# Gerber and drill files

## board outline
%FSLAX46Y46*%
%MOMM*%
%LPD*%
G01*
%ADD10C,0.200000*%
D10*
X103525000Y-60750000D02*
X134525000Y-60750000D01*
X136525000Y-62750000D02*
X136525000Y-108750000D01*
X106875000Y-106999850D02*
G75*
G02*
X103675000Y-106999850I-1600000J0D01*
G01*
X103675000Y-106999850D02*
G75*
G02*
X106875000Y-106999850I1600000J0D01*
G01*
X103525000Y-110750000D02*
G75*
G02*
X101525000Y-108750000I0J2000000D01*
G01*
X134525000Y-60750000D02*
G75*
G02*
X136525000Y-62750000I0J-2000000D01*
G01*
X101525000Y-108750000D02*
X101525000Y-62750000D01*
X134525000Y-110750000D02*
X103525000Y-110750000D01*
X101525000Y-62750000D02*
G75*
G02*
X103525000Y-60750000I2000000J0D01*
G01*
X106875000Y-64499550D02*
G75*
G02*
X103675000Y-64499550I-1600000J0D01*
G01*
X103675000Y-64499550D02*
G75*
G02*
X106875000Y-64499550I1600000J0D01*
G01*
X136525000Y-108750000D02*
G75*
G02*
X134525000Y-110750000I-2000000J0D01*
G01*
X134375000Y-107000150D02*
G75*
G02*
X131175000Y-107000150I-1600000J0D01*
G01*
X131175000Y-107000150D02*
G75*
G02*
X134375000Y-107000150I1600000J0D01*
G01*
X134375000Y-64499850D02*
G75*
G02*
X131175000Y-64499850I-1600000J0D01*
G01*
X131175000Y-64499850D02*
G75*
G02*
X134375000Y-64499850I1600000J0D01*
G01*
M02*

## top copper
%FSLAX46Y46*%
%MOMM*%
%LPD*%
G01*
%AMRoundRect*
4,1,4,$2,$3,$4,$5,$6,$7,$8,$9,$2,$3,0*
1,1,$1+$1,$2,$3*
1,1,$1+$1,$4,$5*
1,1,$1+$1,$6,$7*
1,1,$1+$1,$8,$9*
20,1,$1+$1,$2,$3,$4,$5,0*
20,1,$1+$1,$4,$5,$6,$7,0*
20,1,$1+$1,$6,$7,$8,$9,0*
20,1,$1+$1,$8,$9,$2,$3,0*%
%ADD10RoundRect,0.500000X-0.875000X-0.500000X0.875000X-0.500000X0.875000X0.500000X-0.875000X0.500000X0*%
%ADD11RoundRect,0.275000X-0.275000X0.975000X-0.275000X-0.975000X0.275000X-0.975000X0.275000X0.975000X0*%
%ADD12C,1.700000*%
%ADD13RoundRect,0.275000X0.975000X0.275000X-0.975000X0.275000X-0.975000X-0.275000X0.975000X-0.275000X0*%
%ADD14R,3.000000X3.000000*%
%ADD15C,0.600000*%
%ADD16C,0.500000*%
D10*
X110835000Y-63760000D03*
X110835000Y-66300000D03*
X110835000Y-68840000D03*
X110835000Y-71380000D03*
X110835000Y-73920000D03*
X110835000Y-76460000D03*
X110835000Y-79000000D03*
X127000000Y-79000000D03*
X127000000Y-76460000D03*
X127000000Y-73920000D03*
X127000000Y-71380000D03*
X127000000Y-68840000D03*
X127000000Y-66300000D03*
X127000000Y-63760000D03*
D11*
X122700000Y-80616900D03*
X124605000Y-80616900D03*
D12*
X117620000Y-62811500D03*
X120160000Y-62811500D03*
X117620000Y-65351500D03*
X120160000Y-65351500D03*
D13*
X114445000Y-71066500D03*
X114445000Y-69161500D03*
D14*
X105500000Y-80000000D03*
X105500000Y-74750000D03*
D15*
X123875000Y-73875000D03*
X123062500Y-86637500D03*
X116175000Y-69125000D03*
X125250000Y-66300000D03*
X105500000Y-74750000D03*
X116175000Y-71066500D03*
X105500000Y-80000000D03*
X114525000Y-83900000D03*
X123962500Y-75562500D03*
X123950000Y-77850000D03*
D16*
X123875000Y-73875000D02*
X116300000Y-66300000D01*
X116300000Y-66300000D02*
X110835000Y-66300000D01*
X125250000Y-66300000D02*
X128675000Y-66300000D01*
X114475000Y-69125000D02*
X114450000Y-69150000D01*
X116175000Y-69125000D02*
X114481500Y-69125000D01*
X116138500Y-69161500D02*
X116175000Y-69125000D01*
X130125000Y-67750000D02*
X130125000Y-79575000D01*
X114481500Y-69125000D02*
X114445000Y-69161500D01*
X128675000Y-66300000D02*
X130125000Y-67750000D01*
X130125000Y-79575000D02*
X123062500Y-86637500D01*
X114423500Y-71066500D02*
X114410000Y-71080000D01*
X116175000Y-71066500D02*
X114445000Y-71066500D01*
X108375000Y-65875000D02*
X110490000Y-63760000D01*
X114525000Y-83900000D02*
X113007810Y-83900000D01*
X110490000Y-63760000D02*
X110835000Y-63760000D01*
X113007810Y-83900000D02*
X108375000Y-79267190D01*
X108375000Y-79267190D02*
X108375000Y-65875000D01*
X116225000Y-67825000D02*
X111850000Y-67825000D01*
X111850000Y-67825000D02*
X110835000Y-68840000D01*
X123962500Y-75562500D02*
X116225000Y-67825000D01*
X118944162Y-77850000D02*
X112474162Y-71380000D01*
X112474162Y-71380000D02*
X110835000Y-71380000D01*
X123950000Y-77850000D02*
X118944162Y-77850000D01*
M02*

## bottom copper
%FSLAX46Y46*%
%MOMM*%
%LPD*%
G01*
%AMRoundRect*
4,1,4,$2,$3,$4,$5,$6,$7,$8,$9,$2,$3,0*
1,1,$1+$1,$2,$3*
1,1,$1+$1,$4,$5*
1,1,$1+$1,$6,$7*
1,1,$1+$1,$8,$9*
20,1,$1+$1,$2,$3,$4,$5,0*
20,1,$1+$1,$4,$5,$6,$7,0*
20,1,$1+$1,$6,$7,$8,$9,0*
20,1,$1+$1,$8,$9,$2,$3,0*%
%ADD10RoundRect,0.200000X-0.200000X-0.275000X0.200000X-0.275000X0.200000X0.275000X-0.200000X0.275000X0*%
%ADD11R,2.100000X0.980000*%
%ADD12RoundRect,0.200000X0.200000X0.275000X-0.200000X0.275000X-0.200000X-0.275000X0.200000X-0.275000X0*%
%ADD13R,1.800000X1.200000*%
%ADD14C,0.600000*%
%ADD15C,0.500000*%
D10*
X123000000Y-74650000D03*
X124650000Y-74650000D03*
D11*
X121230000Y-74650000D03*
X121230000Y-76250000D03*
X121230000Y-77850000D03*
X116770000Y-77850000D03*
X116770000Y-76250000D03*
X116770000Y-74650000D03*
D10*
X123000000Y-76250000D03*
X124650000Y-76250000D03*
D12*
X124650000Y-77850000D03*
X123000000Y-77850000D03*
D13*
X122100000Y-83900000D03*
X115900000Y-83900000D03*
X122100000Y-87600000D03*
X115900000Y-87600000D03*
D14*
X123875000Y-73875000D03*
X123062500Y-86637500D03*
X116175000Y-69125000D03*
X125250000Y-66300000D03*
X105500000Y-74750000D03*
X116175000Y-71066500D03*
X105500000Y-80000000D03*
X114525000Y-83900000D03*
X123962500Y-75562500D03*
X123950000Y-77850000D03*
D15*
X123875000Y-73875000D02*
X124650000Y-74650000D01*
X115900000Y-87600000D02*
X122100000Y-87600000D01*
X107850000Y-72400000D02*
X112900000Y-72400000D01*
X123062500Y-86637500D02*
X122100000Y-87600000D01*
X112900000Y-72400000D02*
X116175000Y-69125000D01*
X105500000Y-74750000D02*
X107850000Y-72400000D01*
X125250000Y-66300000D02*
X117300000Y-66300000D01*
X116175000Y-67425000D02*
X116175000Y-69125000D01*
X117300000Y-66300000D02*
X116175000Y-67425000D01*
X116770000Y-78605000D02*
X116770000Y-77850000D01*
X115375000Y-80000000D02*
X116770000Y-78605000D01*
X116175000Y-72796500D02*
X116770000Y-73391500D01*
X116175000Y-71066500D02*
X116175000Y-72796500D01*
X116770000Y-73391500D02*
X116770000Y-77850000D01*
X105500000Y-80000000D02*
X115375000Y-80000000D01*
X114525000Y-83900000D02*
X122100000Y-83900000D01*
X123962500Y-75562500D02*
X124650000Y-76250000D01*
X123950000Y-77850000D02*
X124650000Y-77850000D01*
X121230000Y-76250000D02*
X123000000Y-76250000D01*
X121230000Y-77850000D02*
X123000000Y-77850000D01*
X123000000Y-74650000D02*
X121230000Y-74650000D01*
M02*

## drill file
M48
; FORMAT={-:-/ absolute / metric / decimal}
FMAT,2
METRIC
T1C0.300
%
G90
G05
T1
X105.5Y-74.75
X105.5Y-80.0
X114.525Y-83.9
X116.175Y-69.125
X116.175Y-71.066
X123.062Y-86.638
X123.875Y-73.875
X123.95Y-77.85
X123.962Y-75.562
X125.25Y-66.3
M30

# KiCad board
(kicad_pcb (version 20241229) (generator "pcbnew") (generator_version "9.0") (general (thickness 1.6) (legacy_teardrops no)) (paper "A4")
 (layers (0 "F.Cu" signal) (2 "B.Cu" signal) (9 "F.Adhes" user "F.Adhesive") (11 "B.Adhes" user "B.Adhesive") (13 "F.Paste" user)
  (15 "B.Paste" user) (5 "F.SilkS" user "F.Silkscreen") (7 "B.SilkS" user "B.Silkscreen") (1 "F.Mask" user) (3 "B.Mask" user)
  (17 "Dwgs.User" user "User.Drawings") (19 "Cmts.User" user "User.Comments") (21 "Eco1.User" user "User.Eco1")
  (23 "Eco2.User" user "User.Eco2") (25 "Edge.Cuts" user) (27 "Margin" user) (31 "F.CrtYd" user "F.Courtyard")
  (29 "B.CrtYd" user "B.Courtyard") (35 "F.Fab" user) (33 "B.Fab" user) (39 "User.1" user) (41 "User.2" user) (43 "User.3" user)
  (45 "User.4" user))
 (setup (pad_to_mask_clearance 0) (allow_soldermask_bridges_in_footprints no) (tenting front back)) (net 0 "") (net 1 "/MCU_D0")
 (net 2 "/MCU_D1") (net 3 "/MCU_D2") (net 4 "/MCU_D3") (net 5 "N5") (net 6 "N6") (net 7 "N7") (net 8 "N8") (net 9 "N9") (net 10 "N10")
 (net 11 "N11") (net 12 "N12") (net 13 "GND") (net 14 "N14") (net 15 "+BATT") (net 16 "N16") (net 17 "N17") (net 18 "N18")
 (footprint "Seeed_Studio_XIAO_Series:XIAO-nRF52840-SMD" (layer "F.Cu") (at 110 81.88)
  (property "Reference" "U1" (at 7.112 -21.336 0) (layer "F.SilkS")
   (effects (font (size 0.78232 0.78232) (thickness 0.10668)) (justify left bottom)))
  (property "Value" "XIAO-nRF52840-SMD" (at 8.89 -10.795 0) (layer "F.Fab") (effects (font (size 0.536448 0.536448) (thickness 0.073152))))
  (pad "1" smd roundrect (at 0.835 -18.12) (size 2.75 2) (layers "F.Cu" "F.Mask" "F.Paste") (roundrect_rratio 0.25) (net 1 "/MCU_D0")
   (solder_mask_margin 0.0508) (thermal_bridge_angle 45))
  (pad "2" smd roundrect (at 0.835 -15.58) (size 2.75 2) (layers "F.Cu" "F.Mask" "F.Paste") (roundrect_rratio 0.25) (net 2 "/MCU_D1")
   (solder_mask_margin 0.0508) (thermal_bridge_angle 45))
  (pad "3" smd roundrect (at 0.835 -13.04) (size 2.75 2) (layers "F.Cu" "F.Mask" "F.Paste") (roundrect_rratio 0.25) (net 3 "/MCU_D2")
   (solder_mask_margin 0.0508) (thermal_bridge_angle 45))
  (pad "4" smd roundrect (at 0.835 -10.5) (size 2.75 2) (layers "F.Cu" "F.Mask" "F.Paste") (roundrect_rratio 0.25) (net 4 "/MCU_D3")
   (solder_mask_margin 0.0508) (thermal_bridge_angle 45))
  (pad "5" smd roundrect (at 0.835 -7.96) (size 2.75 2) (layers "F.Cu" "F.Mask" "F.Paste") (roundrect_rratio 0.25) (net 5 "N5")
   (solder_mask_margin 0.0508) (thermal_bridge_angle 45))
  (pad "6" smd roundrect (at 0.835 -5.42) (size 2.75 2) (layers "F.Cu" "F.Mask" "F.Paste") (roundrect_rratio 0.25) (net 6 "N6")
   (solder_mask_margin 0.0508) (thermal_bridge_angle 45))
  (pad "7" smd roundrect (at 0.835 -2.88) (size 2.75 2) (layers "F.Cu" "F.Mask" "F.Paste") (roundrect_rratio 0.25) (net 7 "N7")
   (solder_mask_margin 0.0508) (thermal_bridge_angle 45))
  (pad "8" smd roundrect (at 17 -2.88) (size 2.75 2) (layers "F.Cu" "F.Mask" "F.Paste") (roundrect_rratio 0.25) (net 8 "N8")
   (solder_mask_margin 0.0508) (thermal_bridge_angle 45))
  (pad "9" smd roundrect (at 17 -5.42) (size 2.75 2) (layers "F.Cu" "F.Mask" "F.Paste") (roundrect_rratio 0.25) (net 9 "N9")
   (solder_mask_margin 0.0508) (thermal_bridge_angle 45))
  (pad "10" smd roundrect (at 17 -7.96) (size 2.75 2) (layers "F.Cu" "F.Mask" "F.Paste") (roundrect_rratio 0.25) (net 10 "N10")
   (solder_mask_margin 0.0508) (thermal_bridge_angle 45))
  (pad "11" smd roundrect (at 17 -10.5) (size 2.75 2) (layers "F.Cu" "F.Mask" "F.Paste") (roundrect_rratio 0.25) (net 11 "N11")
   (solder_mask_margin 0.0508) (thermal_bridge_angle 45))
  (pad "12" smd roundrect (at 17 -13.04) (size 2.75 2) (layers "F.Cu" "F.Mask" "F.Paste") (roundrect_rratio 0.25) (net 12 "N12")
   (solder_mask_margin 0.0508) (thermal_bridge_angle 45))
  (pad "13" smd roundrect (at 17 -15.58) (size 2.75 2) (layers "F.Cu" "F.Mask" "F.Paste") (roundrect_rratio 0.25) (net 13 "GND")
   (solder_mask_margin 0.0508) (thermal_bridge_angle 45))
  (pad "14" smd roundrect (at 17 -18.12) (size 2.75 2) (layers "F.Cu" "F.Mask" "F.Paste") (roundrect_rratio 0.25) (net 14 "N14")
   (solder_mask_margin 0.0508) (thermal_bridge_angle 45))
  (pad "17" smd roundrect (at 12.7 -1.2631 270) (size 2.5 1.1) (layers "F.Cu" "F.Mask" "F.Paste") (roundrect_rratio 0.25)
   (solder_mask_margin 0.0508) (thermal_bridge_angle 45))
  (pad "18" smd roundrect (at 14.605 -1.2631 270) (size 2.5 1.1) (layers "F.Cu" "F.Mask" "F.Paste") (roundrect_rratio 0.25)
   (solder_mask_margin 0.0508) (thermal_bridge_angle 45))
  (pad "19" smd circle (at 7.62 -19.0685) (size 1.7 1.7) (layers "F.Cu" "F.Mask" "F.Paste"))
  (pad "20" smd circle (at 10.16 -19.0685) (size 1.7 1.7) (layers "F.Cu" "F.Mask" "F.Paste"))
  (pad "21" smd circle (at 7.62 -16.5285) (size 1.7 1.7) (layers "F.Cu" "F.Mask" "F.Paste"))
  (pad "22" smd circle (at 10.16 -16.5285) (size 1.7 1.7) (layers "F.Cu" "F.Mask" "F.Paste"))
  (pad "32" smd roundrect (at 4.445 -10.8135 180) (size 2.5 1.1) (layers "F.Cu" "F.Mask" "F.Paste") (roundrect_rratio 0.25) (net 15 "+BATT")
   (solder_mask_margin 0.0508) (thermal_bridge_angle 45))
  (pad "33" smd roundrect (at 4.445 -12.7185 180) (size 2.5 1.1) (layers "F.Cu" "F.Mask" "F.Paste") (roundrect_rratio 0.25) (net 13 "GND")
   (solder_mask_margin 0.0508) (thermal_bridge_angle 45)))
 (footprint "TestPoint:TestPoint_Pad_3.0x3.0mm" (layer "F.Cu") (at 105.5 80 90)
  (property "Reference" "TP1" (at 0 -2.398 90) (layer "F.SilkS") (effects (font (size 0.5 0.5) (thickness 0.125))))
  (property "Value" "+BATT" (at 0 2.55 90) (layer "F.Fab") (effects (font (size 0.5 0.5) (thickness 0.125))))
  (pad "1" smd rect (at 0 0 90) (size 3 3) (layers "F.Cu" "F.Mask") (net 15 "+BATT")))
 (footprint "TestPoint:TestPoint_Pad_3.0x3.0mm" (layer "F.Cu") (at 105.5 74.75 90)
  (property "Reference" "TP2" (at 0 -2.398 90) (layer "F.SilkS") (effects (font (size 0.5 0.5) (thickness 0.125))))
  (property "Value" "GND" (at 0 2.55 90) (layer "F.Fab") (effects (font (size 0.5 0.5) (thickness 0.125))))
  (pad "1" smd rect (at 0 0 90) (size 3 3) (layers "F.Cu" "F.Mask") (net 13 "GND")))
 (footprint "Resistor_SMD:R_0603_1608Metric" (layer "B.Cu") (at 123.825 74.65)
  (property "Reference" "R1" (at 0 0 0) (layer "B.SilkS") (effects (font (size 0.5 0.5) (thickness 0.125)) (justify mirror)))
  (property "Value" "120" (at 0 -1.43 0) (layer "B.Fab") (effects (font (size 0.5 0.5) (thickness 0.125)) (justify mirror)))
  (pad "1" smd roundrect (at -0.825 0) (size 0.8 0.95) (layers "B.Cu" "B.Mask" "B.Paste") (roundrect_rratio 0.25) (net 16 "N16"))
  (pad "2" smd roundrect (at 0.825 0) (size 0.8 0.95) (layers "B.Cu" "B.Mask" "B.Paste") (roundrect_rratio 0.25) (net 2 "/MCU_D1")))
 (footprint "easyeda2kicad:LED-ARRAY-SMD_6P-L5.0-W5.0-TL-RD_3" (layer "B.Cu") (at 119 76.25 180)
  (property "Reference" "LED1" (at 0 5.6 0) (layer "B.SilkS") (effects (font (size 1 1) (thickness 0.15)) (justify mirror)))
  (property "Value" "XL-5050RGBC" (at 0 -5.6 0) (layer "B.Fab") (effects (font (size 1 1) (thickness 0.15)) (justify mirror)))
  (pad "1" smd rect (at -2.23 1.6 180) (size 2.1 0.98) (layers "B.Cu" "B.Mask" "B.Paste") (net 16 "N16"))
  (pad "2" smd rect (at -2.23 0 180) (size 2.1 0.98) (layers "B.Cu" "B.Mask" "B.Paste") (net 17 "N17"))
  (pad "3" smd rect (at -2.23 -1.6 180) (size 2.1 0.98) (layers "B.Cu" "B.Mask" "B.Paste") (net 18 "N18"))
  (pad "4" smd rect (at 2.23 -1.6 180) (size 2.1 0.98) (layers "B.Cu" "B.Mask" "B.Paste") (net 15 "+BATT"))
  (pad "5" smd rect (at 2.23 0 180) (size 2.1 0.98) (layers "B.Cu" "B.Mask" "B.Paste") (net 15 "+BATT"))
  (pad "6" smd rect (at 2.23 1.6 180) (size 2.1 0.98) (layers "B.Cu" "B.Mask" "B.Paste") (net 15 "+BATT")))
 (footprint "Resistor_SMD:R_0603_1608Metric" (layer "B.Cu") (at 123.825 76.25)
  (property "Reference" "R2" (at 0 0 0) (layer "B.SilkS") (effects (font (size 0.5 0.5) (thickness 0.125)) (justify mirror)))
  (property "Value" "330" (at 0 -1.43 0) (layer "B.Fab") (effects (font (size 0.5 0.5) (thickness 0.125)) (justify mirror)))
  (pad "1" smd roundrect (at -0.825 0) (size 0.8 0.95) (layers "B.Cu" "B.Mask" "B.Paste") (roundrect_rratio 0.25) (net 17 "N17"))
  (pad "2" smd roundrect (at 0.825 0) (size 0.8 0.95) (layers "B.Cu" "B.Mask" "B.Paste") (roundrect_rratio 0.25) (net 3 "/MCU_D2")))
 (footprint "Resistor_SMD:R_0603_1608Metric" (layer "B.Cu") (at 123.825 77.85 180)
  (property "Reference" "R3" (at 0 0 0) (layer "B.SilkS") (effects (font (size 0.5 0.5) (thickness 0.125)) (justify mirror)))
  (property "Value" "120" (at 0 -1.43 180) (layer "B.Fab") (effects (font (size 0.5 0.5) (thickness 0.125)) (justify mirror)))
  (pad "1" smd roundrect (at -0.825 0 180) (size 0.8 0.95) (layers "B.Cu" "B.Mask" "B.Paste") (roundrect_rratio 0.25) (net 4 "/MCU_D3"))
  (pad "2" smd roundrect (at 0.825 0 180) (size 0.8 0.95) (layers "B.Cu" "B.Mask" "B.Paste") (roundrect_rratio 0.25) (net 18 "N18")))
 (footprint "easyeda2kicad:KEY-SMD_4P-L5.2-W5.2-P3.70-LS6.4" (layer "B.Cu") (at 119 85.75 180)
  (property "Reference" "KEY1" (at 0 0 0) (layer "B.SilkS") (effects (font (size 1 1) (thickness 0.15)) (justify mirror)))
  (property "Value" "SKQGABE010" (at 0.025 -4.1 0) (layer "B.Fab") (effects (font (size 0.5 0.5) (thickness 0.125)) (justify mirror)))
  (pad "1" smd rect (at -3.1 1.85 180) (size 1.8 1.2) (layers "B.Cu" "B.Mask" "B.Paste") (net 1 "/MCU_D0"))
  (pad "2" smd rect (at 3.1 1.85 180) (size 1.8 1.2) (layers "B.Cu" "B.Mask" "B.Paste") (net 1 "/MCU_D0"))
  (pad "3" smd rect (at -3.1 -1.85 180) (size 1.8 1.2) (layers "B.Cu" "B.Mask" "B.Paste") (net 13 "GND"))
  (pad "4" smd rect (at 3.1 -1.85 180) (size 1.8 1.2) (layers "B.Cu" "B.Mask" "B.Paste") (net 13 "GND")))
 (gr_line (start 103.525 60.75) (end 134.525 60.75) (stroke (width 0.2) (type default)) (layer "Edge.Cuts"))
 (gr_line (start 136.525 62.75) (end 136.525 108.75) (stroke (width 0.2) (type default)) (layer "Edge.Cuts"))
 (gr_circle (center 105.275 106.99985) (end 106.875 106.99985) (stroke (width 0.2) (type solid)) (fill no) (layer "Edge.Cuts"))
 (gr_arc (start 103.525 110.75) (mid 102.110786 110.164214) (end 101.525 108.75) (stroke (width 0.2) (type default)) (layer "Edge.Cuts"))
 (gr_arc (start 134.525 60.75) (mid 135.939214 61.335786) (end 136.525 62.75) (stroke (width 0.2) (type default)) (layer "Edge.Cuts"))
 (gr_line (start 101.525 108.75) (end 101.525 62.75) (stroke (width 0.2) (type default)) (layer "Edge.Cuts"))
 (gr_line (start 134.525 110.75) (end 103.525 110.75) (stroke (width 0.2) (type default)) (layer "Edge.Cuts"))
 (gr_arc (start 101.525 62.75) (mid 102.110786 61.335786) (end 103.525 60.75) (stroke (width 0.2) (type default)) (layer "Edge.Cuts"))
 (gr_circle (center 105.275 64.49955) (end 106.875 64.49955) (stroke (width 0.2) (type solid)) (fill no) (layer "Edge.Cuts"))
 (gr_arc (start 136.525 108.75) (mid 135.939214 110.164214) (end 134.525 110.75) (stroke (width 0.2) (type default)) (layer "Edge.Cuts"))
 (gr_circle (center 132.775 107.00015) (end 134.375 107.00015) (stroke (width 0.2) (type solid)) (fill no) (layer "Edge.Cuts"))
 (gr_circle (center 132.775 64.49985) (end 134.375 64.49985) (stroke (width 0.2) (type solid)) (fill no) (layer "Edge.Cuts"))
 (segment (start 123.875 73.875) (end 116.3 66.3) (width 0.5) (layer "F.Cu") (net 2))
 (segment (start 116.3 66.3) (end 110.835 66.3) (width 0.5) (layer "F.Cu") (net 2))
 (via (at 123.875 73.875) (size 0.6) (drill 0.3) (layers "F.Cu" "B.Cu") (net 2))
 (segment (start 123.875 73.875) (end 124.65 74.65) (width 0.5) (layer "B.Cu") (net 2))
 (segment (start 125.25 66.3) (end 128.675 66.3) (width 0.5) (layer "F.Cu") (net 13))
 (segment (start 114.475 69.125) (end 114.45 69.15) (width 0.5) (layer "F.Cu") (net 13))
 (segment (start 116.175 69.125) (end 114.4815 69.125) (width 0.5) (layer "F.Cu") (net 13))
 (segment (start 116.1385 69.1615) (end 116.175 69.125) (width 0.5) (layer "F.Cu") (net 13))
 (segment (start 130.125 67.75) (end 130.125 79.575) (width 0.5) (layer "F.Cu") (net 13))
 (segment (start 114.4815 69.125) (end 114.445 69.1615) (width 0.5) (layer "F.Cu") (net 13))
 (segment (start 128.675 66.3) (end 130.125 67.75) (width 0.5) (layer "F.Cu") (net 13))
 (segment (start 130.125 79.575) (end 123.0625 86.6375) (width 0.5) (layer "F.Cu") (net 13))
 (via (at 123.0625 86.6375) (size 0.6) (drill 0.3) (layers "F.Cu" "B.Cu") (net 13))
 (via (at 116.175 69.125) (size 0.6) (drill 0.3) (layers "F.Cu" "B.Cu") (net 13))
 (via (at 125.25 66.3) (size 0.6) (drill 0.3) (layers "F.Cu" "B.Cu") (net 13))
 (via (at 105.5 74.75) (size 0.6) (drill 0.3) (layers "F.Cu" "B.Cu") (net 13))
 (segment (start 115.9 87.6) (end 122.1 87.6) (width 0.5) (layer "B.Cu") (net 13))
 (segment (start 107.85 72.4) (end 112.9 72.4) (width 0.5) (layer "B.Cu") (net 13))
 (segment (start 123.0625 86.6375) (end 122.1 87.6) (width 0.5) (layer "B.Cu") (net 13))
 (segment (start 112.9 72.4) (end 116.175 69.125) (width 0.5) (layer "B.Cu") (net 13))
 (segment (start 105.5 74.75) (end 107.85 72.4) (width 0.5) (layer "B.Cu") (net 13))
 (segment (start 125.25 66.3) (end 117.3 66.3) (width 0.5) (layer "B.Cu") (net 13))
 (segment (start 116.175 67.425) (end 116.175 69.125) (width 0.5) (layer "B.Cu") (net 13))
 (segment (start 117.3 66.3) (end 116.175 67.425) (width 0.5) (layer "B.Cu") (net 13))
 (segment (start 114.4235 71.0665) (end 114.41 71.08) (width 0.5) (layer "F.Cu") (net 15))
 (segment (start 116.175 71.0665) (end 114.445 71.0665) (width 0.5) (layer "F.Cu") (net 15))
 (via (at 116.175 71.0665) (size 0.6) (drill 0.3) (layers "F.Cu" "B.Cu") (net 15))
 (via (at 105.5 80) (size 0.6) (drill 0.3) (layers "F.Cu" "B.Cu") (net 15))
 (segment (start 116.77 78.605) (end 116.77 77.85) (width 0.5) (layer "B.Cu") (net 15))
 (segment (start 115.375 80) (end 116.77 78.605) (width 0.5) (layer "B.Cu") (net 15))
 (segment (start 116.175 72.7965) (end 116.77 73.3915) (width 0.5) (layer "B.Cu") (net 15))
 (segment (start 116.175 71.0665) (end 116.175 72.7965) (width 0.5) (layer "B.Cu") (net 15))
 (segment (start 116.77 73.3915) (end 116.77 77.85) (width 0.5) (layer "B.Cu") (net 15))
 (segment (start 105.5 80) (end 115.375 80) (width 0.5) (layer "B.Cu") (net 15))
 (segment (start 108.375 65.875) (end 110.49 63.76) (width 0.5) (layer "F.Cu") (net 1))
 (segment (start 114.525 83.9) (end 113.00781 83.9) (width 0.5) (layer "F.Cu") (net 1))
 (segment (start 110.49 63.76) (end 110.835 63.76) (width 0.5) (layer "F.Cu") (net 1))
 (segment (start 113.00781 83.9) (end 108.375 79.26719) (width 0.5) (layer "F.Cu") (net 1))
 (segment (start 108.375 79.26719) (end 108.375 65.875) (width 0.5) (layer "F.Cu") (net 1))
 (via (at 114.525 83.9) (size 0.6) (drill 0.3) (layers "F.Cu" "B.Cu") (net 1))
 (segment (start 114.525 83.9) (end 122.1 83.9) (width 0.5) (layer "B.Cu") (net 1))
 (segment (start 116.225 67.825) (end 111.85 67.825) (width 0.5) (layer "F.Cu") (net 3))
 (segment (start 111.85 67.825) (end 110.835 68.84) (width 0.5) (layer "F.Cu") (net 3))
 (segment (start 123.9625 75.5625) (end 116.225 67.825) (width 0.5) (layer "F.Cu") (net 3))
 (via (at 123.9625 75.5625) (size 0.6) (drill 0.3) (layers "F.Cu" "B.Cu") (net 3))
 (segment (start 123.9625 75.5625) (end 124.65 76.25) (width 0.5) (layer "B.Cu") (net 3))
 (segment (start 118.944162 77.85) (end 112.474162 71.38) (width 0.5) (layer "F.Cu") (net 4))
 (segment (start 112.474162 71.38) (end 110.835 71.38) (width 0.5) (layer "F.Cu") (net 4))
 (segment (start 123.95 77.85) (end 118.944162 77.85) (width 0.5) (layer "F.Cu") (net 4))
 (via (at 123.95 77.85) (size 0.6) (drill 0.3) (layers "F.Cu" "B.Cu") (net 4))
 (segment (start 123.95 77.85) (end 124.65 77.85) (width 0.5) (layer "B.Cu") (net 4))
 (segment (start 121.23 76.25) (end 123 76.25) (width 0.5) (layer "B.Cu") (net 17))
 (segment (start 121.23 77.85) (end 123 77.85) (width 0.5) (layer "B.Cu") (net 18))
 (segment (start 123 74.65) (end 121.23 74.65) (width 0.5) (layer "B.Cu") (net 16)))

